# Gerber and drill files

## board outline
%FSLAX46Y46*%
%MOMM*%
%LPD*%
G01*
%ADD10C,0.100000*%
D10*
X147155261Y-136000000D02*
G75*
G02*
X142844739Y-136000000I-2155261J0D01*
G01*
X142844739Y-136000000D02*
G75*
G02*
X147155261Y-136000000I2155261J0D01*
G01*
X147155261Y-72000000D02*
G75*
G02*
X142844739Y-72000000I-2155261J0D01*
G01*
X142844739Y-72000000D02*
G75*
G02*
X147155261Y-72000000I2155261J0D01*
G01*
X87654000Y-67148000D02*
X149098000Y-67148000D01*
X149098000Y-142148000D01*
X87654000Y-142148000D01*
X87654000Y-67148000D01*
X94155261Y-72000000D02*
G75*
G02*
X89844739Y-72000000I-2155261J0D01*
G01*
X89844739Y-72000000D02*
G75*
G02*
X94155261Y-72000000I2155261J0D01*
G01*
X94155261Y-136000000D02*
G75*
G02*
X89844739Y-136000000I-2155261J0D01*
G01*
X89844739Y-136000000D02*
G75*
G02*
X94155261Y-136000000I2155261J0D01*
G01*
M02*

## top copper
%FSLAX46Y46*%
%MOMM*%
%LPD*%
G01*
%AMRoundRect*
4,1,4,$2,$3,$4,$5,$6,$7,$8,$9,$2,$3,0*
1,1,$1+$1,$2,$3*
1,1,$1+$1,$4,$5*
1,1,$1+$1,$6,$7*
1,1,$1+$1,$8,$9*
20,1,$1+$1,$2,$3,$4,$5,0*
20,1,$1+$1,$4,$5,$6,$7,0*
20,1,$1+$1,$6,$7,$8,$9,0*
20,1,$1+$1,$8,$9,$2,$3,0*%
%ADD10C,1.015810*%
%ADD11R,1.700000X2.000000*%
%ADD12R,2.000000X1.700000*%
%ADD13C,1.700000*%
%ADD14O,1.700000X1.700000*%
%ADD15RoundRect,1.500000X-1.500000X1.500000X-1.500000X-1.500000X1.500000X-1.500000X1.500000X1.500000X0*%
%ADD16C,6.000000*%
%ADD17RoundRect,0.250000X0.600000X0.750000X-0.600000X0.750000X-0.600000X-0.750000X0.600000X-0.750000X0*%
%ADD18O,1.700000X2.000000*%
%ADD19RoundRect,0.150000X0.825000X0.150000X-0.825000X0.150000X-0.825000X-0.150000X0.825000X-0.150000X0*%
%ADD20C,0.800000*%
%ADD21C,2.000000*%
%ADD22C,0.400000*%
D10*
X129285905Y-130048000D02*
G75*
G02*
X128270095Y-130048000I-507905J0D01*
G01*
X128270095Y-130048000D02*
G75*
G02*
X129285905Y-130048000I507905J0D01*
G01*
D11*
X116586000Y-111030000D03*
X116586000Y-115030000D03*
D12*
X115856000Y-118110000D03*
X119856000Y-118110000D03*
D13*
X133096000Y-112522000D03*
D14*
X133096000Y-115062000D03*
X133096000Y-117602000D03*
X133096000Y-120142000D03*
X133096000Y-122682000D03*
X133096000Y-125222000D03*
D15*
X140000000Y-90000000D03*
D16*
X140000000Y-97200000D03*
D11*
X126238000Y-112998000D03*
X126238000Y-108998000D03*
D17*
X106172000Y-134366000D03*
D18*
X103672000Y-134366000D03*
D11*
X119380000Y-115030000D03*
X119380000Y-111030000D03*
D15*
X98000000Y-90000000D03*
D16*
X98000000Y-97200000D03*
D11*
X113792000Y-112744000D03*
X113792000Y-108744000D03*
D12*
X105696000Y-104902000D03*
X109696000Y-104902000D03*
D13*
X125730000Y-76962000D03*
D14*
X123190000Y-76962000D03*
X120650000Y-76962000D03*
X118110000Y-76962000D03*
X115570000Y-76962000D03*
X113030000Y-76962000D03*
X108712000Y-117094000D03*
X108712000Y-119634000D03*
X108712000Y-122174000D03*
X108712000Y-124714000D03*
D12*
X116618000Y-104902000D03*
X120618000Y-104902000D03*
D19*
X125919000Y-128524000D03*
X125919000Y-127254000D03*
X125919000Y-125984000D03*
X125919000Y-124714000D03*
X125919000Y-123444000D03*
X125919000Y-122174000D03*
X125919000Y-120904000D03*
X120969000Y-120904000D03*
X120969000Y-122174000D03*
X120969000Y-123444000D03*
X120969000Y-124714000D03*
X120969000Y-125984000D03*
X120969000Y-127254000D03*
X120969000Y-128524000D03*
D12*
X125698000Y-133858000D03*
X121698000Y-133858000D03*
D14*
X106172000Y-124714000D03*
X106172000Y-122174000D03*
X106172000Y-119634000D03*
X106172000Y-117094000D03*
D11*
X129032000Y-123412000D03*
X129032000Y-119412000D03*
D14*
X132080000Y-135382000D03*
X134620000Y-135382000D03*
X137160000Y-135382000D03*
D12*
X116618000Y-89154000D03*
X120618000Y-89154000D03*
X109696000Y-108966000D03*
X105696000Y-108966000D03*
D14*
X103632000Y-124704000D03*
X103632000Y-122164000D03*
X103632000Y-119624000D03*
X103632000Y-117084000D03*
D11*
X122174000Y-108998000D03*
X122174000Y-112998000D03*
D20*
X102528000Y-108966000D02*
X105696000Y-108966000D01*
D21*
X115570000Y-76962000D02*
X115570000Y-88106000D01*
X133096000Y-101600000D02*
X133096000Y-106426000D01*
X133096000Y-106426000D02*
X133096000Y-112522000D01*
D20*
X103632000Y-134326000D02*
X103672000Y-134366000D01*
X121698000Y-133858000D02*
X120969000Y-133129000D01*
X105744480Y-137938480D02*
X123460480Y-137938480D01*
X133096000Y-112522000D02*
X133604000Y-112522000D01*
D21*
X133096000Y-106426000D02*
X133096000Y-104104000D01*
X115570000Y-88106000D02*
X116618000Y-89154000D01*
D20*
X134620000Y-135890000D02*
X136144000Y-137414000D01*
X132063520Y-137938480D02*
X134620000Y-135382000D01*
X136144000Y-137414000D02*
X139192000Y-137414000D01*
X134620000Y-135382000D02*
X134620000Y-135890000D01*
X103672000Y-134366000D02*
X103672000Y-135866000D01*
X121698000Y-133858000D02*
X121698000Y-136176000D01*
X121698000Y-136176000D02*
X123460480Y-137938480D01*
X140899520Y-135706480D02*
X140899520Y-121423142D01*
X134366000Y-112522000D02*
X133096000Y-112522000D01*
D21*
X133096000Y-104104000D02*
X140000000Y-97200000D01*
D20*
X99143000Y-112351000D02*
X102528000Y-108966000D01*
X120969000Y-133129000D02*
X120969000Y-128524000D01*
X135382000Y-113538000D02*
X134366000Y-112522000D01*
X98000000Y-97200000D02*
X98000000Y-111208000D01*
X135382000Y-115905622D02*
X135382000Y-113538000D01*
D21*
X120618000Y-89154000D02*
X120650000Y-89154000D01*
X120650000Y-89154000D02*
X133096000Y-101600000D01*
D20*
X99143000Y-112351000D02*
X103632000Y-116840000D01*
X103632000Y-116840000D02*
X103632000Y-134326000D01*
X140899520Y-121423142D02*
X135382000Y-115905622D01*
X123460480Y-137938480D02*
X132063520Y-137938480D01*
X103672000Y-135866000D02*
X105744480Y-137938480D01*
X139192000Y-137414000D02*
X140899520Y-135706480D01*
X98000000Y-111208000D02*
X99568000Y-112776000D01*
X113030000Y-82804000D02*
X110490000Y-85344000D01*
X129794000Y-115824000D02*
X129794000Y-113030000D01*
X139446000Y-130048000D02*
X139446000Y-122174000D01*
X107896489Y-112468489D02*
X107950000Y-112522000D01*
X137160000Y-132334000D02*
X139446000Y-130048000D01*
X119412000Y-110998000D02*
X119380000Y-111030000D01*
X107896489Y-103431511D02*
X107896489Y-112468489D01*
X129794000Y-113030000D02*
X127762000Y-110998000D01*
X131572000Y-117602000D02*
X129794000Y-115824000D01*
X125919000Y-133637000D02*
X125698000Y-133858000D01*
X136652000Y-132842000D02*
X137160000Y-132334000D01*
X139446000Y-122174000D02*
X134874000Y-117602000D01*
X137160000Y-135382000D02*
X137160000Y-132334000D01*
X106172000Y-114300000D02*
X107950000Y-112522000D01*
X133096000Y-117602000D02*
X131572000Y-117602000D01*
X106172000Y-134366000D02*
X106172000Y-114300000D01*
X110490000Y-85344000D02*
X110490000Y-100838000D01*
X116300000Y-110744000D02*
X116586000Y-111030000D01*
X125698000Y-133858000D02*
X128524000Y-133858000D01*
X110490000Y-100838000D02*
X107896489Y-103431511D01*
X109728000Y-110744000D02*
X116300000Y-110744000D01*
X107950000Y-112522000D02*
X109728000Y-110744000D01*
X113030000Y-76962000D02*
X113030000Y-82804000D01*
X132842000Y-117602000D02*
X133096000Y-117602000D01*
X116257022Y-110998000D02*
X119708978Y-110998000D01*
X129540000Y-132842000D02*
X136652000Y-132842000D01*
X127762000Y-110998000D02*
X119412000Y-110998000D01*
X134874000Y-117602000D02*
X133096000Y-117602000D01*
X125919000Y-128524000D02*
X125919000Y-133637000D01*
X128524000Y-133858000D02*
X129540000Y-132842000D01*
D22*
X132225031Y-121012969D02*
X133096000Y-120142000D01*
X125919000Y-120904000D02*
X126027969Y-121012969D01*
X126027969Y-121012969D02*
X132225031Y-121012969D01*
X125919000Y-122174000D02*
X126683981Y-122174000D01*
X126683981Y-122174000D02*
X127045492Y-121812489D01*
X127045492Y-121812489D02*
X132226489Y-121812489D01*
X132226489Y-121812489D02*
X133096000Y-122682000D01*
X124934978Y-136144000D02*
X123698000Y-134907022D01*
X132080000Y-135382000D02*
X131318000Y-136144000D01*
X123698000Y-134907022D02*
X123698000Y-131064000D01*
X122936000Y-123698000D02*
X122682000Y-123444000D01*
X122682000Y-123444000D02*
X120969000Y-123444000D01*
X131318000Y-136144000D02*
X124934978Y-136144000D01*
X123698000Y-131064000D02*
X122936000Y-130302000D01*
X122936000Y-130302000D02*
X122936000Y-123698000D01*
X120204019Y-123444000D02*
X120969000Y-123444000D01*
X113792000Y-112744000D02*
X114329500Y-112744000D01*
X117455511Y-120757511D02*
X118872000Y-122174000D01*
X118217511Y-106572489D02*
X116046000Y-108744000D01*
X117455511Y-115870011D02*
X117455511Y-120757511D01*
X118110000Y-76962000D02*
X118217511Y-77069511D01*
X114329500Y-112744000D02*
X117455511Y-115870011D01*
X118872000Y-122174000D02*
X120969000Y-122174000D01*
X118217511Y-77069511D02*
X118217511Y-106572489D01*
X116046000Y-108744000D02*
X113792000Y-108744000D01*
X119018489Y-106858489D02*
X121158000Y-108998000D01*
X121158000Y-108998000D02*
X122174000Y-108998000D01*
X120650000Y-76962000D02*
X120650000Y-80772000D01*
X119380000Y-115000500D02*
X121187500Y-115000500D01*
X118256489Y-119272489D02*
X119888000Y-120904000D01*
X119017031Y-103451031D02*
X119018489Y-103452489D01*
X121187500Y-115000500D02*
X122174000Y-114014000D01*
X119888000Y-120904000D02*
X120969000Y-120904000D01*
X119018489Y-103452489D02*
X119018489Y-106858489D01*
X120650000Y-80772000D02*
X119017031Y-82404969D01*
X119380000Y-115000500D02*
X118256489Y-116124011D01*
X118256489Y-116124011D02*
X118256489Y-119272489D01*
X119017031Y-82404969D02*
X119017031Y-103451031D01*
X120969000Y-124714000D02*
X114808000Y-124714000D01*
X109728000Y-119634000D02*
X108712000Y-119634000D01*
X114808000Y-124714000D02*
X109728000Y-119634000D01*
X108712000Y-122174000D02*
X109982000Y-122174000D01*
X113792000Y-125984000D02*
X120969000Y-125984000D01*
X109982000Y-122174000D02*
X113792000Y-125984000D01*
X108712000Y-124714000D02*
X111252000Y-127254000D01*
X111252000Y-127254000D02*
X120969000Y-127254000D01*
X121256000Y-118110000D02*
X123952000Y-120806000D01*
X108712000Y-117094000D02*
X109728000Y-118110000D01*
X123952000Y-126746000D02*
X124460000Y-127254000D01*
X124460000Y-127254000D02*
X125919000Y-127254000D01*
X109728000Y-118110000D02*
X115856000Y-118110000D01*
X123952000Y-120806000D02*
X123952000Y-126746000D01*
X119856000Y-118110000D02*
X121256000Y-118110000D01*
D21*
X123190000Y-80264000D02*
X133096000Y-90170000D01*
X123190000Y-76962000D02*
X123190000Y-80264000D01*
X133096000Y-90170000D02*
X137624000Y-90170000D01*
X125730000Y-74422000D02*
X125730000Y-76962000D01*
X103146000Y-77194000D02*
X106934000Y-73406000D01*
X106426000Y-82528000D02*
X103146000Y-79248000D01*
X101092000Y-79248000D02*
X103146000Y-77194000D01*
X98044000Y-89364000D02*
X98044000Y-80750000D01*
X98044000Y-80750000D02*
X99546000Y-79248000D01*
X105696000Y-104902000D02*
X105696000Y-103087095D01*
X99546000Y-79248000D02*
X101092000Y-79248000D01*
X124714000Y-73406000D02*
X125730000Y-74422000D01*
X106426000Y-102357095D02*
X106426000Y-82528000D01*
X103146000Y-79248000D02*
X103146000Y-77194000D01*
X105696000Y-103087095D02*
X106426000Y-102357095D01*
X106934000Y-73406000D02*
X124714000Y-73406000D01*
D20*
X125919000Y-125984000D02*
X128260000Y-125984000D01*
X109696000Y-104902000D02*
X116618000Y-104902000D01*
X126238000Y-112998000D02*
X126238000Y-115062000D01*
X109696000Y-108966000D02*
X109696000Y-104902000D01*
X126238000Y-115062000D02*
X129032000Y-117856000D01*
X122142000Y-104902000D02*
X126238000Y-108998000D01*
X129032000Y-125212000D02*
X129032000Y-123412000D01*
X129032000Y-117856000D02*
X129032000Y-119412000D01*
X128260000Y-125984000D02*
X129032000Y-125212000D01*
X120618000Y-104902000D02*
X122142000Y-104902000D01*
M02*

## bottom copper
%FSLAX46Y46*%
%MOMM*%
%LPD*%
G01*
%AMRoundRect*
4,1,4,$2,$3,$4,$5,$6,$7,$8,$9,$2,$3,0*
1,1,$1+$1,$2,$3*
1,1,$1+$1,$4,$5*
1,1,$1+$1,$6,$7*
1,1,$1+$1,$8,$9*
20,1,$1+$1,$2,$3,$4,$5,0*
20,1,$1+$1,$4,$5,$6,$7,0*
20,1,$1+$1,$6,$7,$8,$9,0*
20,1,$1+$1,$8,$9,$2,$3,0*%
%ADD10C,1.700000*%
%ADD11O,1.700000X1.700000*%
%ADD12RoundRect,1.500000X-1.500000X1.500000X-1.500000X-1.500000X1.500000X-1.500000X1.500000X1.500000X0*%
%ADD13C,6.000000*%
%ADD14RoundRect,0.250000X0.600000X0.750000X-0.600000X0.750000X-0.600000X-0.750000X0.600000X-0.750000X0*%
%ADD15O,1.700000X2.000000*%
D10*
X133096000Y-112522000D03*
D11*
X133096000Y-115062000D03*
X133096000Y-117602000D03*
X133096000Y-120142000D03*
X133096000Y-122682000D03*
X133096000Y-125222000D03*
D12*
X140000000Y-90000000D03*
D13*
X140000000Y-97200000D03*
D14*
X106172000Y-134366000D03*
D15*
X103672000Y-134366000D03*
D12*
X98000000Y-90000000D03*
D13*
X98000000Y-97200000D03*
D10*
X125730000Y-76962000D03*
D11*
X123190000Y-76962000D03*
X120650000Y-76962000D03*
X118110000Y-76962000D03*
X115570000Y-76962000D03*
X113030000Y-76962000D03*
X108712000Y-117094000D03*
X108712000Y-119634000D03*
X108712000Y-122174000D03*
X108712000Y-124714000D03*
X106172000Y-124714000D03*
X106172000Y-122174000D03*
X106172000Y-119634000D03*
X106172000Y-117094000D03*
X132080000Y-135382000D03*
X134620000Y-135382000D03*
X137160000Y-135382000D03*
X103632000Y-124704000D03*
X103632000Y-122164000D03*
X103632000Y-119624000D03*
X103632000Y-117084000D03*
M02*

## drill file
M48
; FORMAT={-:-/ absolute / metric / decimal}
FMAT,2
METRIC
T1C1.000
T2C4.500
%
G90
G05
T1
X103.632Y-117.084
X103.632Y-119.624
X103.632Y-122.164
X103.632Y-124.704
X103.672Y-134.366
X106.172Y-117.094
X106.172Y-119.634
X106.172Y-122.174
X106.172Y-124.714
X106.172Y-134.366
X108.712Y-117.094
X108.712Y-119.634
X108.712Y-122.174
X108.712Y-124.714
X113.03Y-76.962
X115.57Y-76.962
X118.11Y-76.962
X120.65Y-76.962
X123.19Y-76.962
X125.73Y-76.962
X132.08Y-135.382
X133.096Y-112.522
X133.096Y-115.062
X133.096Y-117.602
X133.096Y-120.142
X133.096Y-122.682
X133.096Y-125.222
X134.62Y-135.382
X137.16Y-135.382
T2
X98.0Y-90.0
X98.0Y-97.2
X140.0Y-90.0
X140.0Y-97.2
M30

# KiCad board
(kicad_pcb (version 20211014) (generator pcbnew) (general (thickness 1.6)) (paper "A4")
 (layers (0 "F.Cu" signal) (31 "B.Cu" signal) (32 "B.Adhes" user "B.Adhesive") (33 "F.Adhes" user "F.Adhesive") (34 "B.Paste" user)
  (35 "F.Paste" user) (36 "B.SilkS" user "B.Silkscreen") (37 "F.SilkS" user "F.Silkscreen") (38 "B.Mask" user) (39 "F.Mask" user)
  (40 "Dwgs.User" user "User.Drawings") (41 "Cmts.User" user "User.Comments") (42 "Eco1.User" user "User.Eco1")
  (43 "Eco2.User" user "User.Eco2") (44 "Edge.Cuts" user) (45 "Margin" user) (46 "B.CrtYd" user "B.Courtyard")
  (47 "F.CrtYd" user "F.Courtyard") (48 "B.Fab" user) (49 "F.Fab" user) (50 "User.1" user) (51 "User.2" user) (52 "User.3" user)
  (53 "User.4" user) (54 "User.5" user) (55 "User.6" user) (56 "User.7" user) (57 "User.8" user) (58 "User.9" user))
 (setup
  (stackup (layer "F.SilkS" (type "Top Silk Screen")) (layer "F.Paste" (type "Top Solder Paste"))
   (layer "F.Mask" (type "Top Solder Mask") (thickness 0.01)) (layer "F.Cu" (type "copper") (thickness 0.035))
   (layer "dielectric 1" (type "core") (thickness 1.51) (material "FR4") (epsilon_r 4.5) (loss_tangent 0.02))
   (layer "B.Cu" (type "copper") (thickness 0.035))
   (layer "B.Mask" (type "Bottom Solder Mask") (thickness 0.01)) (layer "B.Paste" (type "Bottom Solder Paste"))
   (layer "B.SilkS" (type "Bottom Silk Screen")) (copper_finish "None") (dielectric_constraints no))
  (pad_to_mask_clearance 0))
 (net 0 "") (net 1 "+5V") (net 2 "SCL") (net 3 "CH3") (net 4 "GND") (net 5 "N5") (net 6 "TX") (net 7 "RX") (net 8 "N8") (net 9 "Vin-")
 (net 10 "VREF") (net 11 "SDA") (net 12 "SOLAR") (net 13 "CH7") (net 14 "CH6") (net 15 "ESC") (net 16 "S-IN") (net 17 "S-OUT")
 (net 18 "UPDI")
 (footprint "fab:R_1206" (layer "F.Cu") (at 116.586 113.03 -90)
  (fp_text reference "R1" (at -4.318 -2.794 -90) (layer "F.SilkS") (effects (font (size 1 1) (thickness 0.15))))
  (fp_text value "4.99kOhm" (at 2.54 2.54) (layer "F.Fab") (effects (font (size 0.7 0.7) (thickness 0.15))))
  (pad "1" smd rect locked (at -2 0 270) (size 2 1.7) (layers "F.Cu" "F.Paste" "F.Mask") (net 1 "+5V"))
  (pad "2" smd rect locked (at 2 0 270) (size 2 1.7) (layers "F.Cu" "F.Paste" "F.Mask") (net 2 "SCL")))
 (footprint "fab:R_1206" (layer "F.Cu") (at 117.856 118.11)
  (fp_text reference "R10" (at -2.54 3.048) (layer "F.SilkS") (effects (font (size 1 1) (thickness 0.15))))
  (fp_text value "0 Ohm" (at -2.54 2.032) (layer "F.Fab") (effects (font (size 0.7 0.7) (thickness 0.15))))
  (pad "1" smd rect locked (at -2 0) (size 2 1.7) (layers "F.Cu" "F.Paste" "F.Mask") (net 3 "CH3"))
  (pad "2" smd rect locked (at 2 0) (size 2 1.7) (layers "F.Cu" "F.Paste" "F.Mask") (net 3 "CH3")))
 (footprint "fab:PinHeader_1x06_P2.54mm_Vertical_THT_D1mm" (layer "F.Cu") (at 133.096 112.522)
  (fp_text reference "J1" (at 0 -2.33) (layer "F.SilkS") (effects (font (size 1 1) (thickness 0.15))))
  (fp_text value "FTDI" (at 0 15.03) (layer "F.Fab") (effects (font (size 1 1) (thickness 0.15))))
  (pad "1" thru_hole circle locked (at 0 0) (size 1.7 1.7) (drill 1) (layers *.Cu *.Mask) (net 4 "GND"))
  (pad "2" thru_hole oval locked (at 0 2.54) (size 1.7 1.7) (drill 1) (layers *.Cu *.Mask) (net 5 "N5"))
  (pad "3" thru_hole oval locked (at 0 5.08) (size 1.7 1.7) (drill 1) (layers *.Cu *.Mask) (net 1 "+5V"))
  (pad "4" thru_hole oval locked (at 0 7.62) (size 1.7 1.7) (drill 1) (layers *.Cu *.Mask) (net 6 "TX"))
  (pad "5" thru_hole oval locked (at 0 10.16) (size 1.7 1.7) (drill 1) (layers *.Cu *.Mask) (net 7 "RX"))
  (pad "6" thru_hole oval locked (at 0 12.7) (size 1.7 1.7) (drill 1) (layers *.Cu *.Mask) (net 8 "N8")))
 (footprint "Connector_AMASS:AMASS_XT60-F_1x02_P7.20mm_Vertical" (layer "F.Cu") (at 140 90 -90)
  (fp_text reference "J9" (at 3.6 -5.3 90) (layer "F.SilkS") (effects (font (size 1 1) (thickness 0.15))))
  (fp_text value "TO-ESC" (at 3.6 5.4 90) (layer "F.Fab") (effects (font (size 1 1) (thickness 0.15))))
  (pad "1" thru_hole roundrect (at 0 0 270) (size 6 6) (drill 4.5) (layers *.Cu *.Mask) (roundrect_rratio 0.25) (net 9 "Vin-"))
  (pad "2" thru_hole circle (at 7.2 0 270) (size 6 6) (drill 4.5) (layers *.Cu *.Mask) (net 4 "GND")))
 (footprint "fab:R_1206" (layer "F.Cu") (at 126.238 110.998 90)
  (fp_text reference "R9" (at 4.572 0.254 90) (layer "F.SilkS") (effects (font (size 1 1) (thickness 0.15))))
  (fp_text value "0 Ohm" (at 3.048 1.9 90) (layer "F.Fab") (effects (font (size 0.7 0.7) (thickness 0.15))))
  (pad "1" smd rect locked (at -2 0 90) (size 2 1.7) (layers "F.Cu" "F.Paste" "F.Mask") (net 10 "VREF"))
  (pad "2" smd rect locked (at 2 0 90) (size 2 1.7) (layers "F.Cu" "F.Paste" "F.Mask") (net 10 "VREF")))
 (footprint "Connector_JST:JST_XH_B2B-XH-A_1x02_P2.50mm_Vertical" (layer "F.Cu") (at 106.172 134.366 180)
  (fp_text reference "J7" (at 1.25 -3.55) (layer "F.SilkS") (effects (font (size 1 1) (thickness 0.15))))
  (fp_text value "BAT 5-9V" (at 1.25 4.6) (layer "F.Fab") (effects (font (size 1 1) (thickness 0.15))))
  (pad "1" thru_hole roundrect (at 0 0 180) (size 1.7 2) (drill 1) (layers *.Cu *.Mask) (roundrect_rratio 0.1470588235) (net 1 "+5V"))
  (pad "2" thru_hole oval (at 2.5 0 180) (size 1.7 2) (drill 1) (layers *.Cu *.Mask) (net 4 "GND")))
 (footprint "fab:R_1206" (layer "F.Cu") (at 119.38 113.03 90)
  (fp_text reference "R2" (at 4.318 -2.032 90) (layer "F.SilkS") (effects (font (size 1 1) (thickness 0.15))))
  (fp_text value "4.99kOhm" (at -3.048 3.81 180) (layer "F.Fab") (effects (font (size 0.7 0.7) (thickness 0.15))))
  (pad "1" smd rect locked (at -2 0 90) (size 2 1.7) (layers "F.Cu" "F.Paste" "F.Mask") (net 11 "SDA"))
  (pad "2" smd rect locked (at 2 0 90) (size 2 1.7) (layers "F.Cu" "F.Paste" "F.Mask") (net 1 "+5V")))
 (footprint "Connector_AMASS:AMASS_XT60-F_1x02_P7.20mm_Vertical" (layer "F.Cu") (at 98 90 -90)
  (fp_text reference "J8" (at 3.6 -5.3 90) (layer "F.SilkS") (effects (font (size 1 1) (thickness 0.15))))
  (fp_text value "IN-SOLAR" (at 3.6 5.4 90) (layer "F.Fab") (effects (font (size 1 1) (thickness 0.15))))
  (pad "1" thru_hole roundrect (at 0 0 270) (size 6 6) (drill 4.5) (layers *.Cu *.Mask) (roundrect_rratio 0.25) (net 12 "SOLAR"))
  (pad "2" thru_hole circle (at 7.2 0 270) (size 6 6) (drill 4.5) (layers *.Cu *.Mask) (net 4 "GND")))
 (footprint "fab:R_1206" (layer "F.Cu") (at 113.792 110.744 90)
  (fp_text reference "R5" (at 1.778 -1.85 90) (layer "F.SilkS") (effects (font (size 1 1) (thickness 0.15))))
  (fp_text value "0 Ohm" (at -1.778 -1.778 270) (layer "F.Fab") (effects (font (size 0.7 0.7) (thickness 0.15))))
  (pad "1" smd rect locked (at -2 0 90) (size 2 1.7) (layers "F.Cu" "F.Paste" "F.Mask") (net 2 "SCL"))
  (pad "2" smd rect locked (at 2 0 90) (size 2 1.7) (layers "F.Cu" "F.Paste" "F.Mask") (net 2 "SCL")))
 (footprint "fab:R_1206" (layer "F.Cu") (at 107.696 104.902)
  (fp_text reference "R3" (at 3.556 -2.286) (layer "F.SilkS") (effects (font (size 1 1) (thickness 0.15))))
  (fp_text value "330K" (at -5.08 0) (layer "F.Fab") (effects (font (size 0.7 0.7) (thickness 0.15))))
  (pad "1" smd rect locked (at -2 0) (size 2 1.7) (layers "F.Cu" "F.Paste" "F.Mask") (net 12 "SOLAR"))
  (pad "2" smd rect locked (at 2 0) (size 2 1.7) (layers "F.Cu" "F.Paste" "F.Mask") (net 10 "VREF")))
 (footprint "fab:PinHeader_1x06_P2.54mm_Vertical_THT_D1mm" (layer "F.Cu") (at 125.73 76.962 -90)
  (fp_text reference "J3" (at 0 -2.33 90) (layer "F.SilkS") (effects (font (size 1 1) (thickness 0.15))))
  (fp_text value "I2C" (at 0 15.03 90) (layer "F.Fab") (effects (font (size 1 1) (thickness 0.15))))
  (pad "1" thru_hole circle locked (at 0 0 270) (size 1.7 1.7) (drill 1) (layers *.Cu *.Mask) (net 12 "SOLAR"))
  (pad "2" thru_hole oval locked (at 0 2.54 270) (size 1.7 1.7) (drill 1) (layers *.Cu *.Mask) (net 9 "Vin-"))
  (pad "3" thru_hole oval locked (at 0 5.08 270) (size 1.7 1.7) (drill 1) (layers *.Cu *.Mask) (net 11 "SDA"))
  (pad "4" thru_hole oval locked (at 0 7.62 270) (size 1.7 1.7) (drill 1) (layers *.Cu *.Mask) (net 2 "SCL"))
  (pad "5" thru_hole oval locked (at 0 10.16 270) (size 1.7 1.7) (drill 1) (layers *.Cu *.Mask) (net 4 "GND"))
  (pad "6" thru_hole oval locked (at 0 12.7 270) (size 1.7 1.7) (drill 1) (layers *.Cu *.Mask) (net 1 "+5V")))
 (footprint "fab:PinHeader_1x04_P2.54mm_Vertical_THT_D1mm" (layer "F.Cu") (at 108.712 117.094)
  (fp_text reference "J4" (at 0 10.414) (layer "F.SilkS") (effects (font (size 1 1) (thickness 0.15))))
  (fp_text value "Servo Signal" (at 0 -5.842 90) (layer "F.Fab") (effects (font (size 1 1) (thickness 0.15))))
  (pad "1" thru_hole oval locked (at 0 0) (size 1.7 1.7) (drill 1) (layers *.Cu *.Mask) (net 3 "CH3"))
  (pad "2" thru_hole oval locked (at 0 2.54) (size 1.7 1.7) (drill 1) (layers *.Cu *.Mask) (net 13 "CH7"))
  (pad "3" thru_hole oval locked (at 0 5.08) (size 1.7 1.7) (drill 1) (layers *.Cu *.Mask) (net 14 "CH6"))
  (pad "4" thru_hole oval locked (at 0 7.62) (size 1.7 1.7) (drill 1) (layers *.Cu *.Mask) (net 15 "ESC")))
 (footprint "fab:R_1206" (layer "F.Cu") (at 118.618 104.902)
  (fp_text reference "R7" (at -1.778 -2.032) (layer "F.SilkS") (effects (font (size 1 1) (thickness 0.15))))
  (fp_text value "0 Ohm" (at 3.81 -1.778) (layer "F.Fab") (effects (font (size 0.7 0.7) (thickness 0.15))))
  (pad "1" smd rect locked (at -2 0) (size 2 1.7) (layers "F.Cu" "F.Paste" "F.Mask") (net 10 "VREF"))
  (pad "2" smd rect locked (at 2 0) (size 2 1.7) (layers "F.Cu" "F.Paste" "F.Mask") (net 10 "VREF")))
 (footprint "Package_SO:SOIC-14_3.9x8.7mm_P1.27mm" (layer "F.Cu") (at 123.444 124.714 180)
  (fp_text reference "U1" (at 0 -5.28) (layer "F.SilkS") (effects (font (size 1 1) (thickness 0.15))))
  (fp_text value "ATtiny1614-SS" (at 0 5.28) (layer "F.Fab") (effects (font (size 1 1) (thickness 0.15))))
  (pad "1" smd roundrect (at -2.475 -3.81 180) (size 1.95 0.6) (layers "F.Cu" "F.Paste" "F.Mask") (roundrect_rratio 0.25) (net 1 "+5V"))
  (pad "2" smd roundrect (at -2.475 -2.54 180) (size 1.95 0.6) (layers "F.Cu" "F.Paste" "F.Mask") (roundrect_rratio 0.25) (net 3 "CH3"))
  (pad "3" smd roundrect (at -2.475 -1.27 180) (size 1.95 0.6) (layers "F.Cu" "F.Paste" "F.Mask") (roundrect_rratio 0.25) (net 10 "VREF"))
  (pad "4" smd roundrect (at -2.475 0 180) (size 1.95 0.6) (layers "F.Cu" "F.Paste" "F.Mask") (roundrect_rratio 0.25) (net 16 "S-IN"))
  (pad "5" smd roundrect (at -2.475 1.27 180) (size 1.95 0.6) (layers "F.Cu" "F.Paste" "F.Mask") (roundrect_rratio 0.25) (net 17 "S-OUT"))
  (pad "6" smd roundrect (at -2.475 2.54 180) (size 1.95 0.6) (layers "F.Cu" "F.Paste" "F.Mask") (roundrect_rratio 0.25) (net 7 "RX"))
  (pad "7" smd roundrect (at -2.475 3.81 180) (size 1.95 0.6) (layers "F.Cu" "F.Paste" "F.Mask") (roundrect_rratio 0.25) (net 6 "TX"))
  (pad "8" smd roundrect (at 2.475 3.81 180) (size 1.95 0.6) (layers "F.Cu" "F.Paste" "F.Mask") (roundrect_rratio 0.25) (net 11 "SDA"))
  (pad "9" smd roundrect (at 2.475 2.54 180) (size 1.95 0.6) (layers "F.Cu" "F.Paste" "F.Mask") (roundrect_rratio 0.25) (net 2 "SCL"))
  (pad "10" smd roundrect (at 2.475 1.27 180) (size 1.95 0.6) (layers "F.Cu" "F.Paste" "F.Mask") (roundrect_rratio 0.25) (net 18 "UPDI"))
  (pad "11" smd roundrect (at 2.475 0 180) (size 1.95 0.6) (layers "F.Cu" "F.Paste" "F.Mask") (roundrect_rratio 0.25) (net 13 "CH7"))
  (pad "12" smd roundrect (at 2.475 -1.27 180) (size 1.95 0.6) (layers "F.Cu" "F.Paste" "F.Mask") (roundrect_rratio 0.25) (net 14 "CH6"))
  (pad "13" smd roundrect (at 2.475 -2.54 180) (size 1.95 0.6) (layers "F.Cu" "F.Paste" "F.Mask") (roundrect_rratio 0.25) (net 15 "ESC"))
  (pad "14" smd roundrect (at 2.475 -3.81 180) (size 1.95 0.6) (layers "F.Cu" "F.Paste" "F.Mask") (roundrect_rratio 0.25) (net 4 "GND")))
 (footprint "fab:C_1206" (layer "F.Cu") (at 123.698 133.858 180)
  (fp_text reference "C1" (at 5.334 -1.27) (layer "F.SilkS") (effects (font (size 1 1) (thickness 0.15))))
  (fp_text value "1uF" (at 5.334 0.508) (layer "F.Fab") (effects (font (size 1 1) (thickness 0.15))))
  (pad "1" smd rect locked (at -2 0 180) (size 2 1.7) (layers "F.Cu" "F.Paste" "F.Mask") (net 1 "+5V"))
  (pad "2" smd rect locked (at 2 0 180) (size 2 1.7) (layers "F.Cu" "F.Paste" "F.Mask") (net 4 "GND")))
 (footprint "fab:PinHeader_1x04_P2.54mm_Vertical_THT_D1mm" (layer "F.Cu") (at 106.172 124.714 180)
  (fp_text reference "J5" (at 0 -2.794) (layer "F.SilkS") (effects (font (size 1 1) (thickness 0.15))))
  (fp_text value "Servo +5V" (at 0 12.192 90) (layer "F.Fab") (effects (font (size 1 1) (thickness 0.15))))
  (pad "1" thru_hole oval locked (at 0 0 180) (size 1.7 1.7) (drill 1) (layers *.Cu *.Mask) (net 1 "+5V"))
  (pad "2" thru_hole oval locked (at 0 2.54 180) (size 1.7 1.7) (drill 1) (layers *.Cu *.Mask) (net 1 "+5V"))
  (pad "3" thru_hole oval locked (at 0 5.08 180) (size 1.7 1.7) (drill 1) (layers *.Cu *.Mask) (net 1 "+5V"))
  (pad "4" thru_hole oval locked (at 0 7.62 180) (size 1.7 1.7) (drill 1) (layers *.Cu *.Mask) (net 1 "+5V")))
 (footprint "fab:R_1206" (layer "F.Cu") (at 129.032 121.412 90)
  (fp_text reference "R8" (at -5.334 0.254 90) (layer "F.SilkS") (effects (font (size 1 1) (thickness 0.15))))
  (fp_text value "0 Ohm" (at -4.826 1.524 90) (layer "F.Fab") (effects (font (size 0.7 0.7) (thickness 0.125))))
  (pad "1" smd rect locked (at -2 0 90) (size 2 1.7) (layers "F.Cu" "F.Paste" "F.Mask") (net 10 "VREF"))
  (pad "2" smd rect locked (at 2 0 90) (size 2 1.7) (layers "F.Cu" "F.Paste" "F.Mask") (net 10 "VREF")))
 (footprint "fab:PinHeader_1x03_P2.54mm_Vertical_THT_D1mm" (layer "F.Cu") (at 132.08 135.382 90)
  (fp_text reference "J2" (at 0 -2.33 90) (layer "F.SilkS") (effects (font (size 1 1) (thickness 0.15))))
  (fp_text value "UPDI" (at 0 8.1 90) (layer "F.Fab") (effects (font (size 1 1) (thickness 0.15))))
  (pad "1" thru_hole oval locked (at 0 0 90) (size 1.7 1.7) (drill 1) (layers *.Cu *.Mask) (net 18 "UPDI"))
  (pad "2" thru_hole oval locked (at 0 2.54 90) (size 1.7 1.7) (drill 1) (layers *.Cu *.Mask) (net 4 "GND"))
  (pad "3" thru_hole oval locked (at 0 5.08 90) (size 1.7 1.7) (drill 1) (layers *.Cu *.Mask) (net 1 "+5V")))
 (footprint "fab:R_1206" (layer "F.Cu") (at 118.618 89.154)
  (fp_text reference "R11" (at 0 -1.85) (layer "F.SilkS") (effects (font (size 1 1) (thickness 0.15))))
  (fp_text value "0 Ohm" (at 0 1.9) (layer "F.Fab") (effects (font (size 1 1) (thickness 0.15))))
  (pad "1" smd rect locked (at -2 0) (size 2 1.7) (layers "F.Cu" "F.Paste" "F.Mask") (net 4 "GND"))
  (pad "2" smd rect locked (at 2 0) (size 2 1.7) (layers "F.Cu" "F.Paste" "F.Mask") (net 4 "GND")))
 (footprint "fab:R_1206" (layer "F.Cu") (at 107.696 108.966 180)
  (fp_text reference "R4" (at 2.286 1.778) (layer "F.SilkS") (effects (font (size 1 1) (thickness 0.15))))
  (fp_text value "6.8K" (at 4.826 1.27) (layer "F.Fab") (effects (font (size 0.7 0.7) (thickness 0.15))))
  (pad "1" smd rect locked (at -2 0 180) (size 2 1.7) (layers "F.Cu" "F.Paste" "F.Mask") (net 10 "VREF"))
  (pad "2" smd rect locked (at 2 0 180) (size 2 1.7) (layers "F.Cu" "F.Paste" "F.Mask") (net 4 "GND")))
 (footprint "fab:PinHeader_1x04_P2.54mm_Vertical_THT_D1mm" (layer "F.Cu") (at 103.632 124.704 180)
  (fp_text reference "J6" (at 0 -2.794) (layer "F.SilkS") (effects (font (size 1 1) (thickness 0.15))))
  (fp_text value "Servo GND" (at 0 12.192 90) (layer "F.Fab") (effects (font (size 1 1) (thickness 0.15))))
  (pad "1" thru_hole oval locked (at 0 0 180) (size 1.7 1.7) (drill 1) (layers *.Cu *.Mask) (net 4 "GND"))
  (pad "2" thru_hole oval locked (at 0 2.54 180) (size 1.7 1.7) (drill 1) (layers *.Cu *.Mask) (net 4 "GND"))
  (pad "3" thru_hole oval locked (at 0 5.08 180) (size 1.7 1.7) (drill 1) (layers *.Cu *.Mask) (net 4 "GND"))
  (pad "4" thru_hole oval locked (at 0 7.62 180) (size 1.7 1.7) (drill 1) (layers *.Cu *.Mask) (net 4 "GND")))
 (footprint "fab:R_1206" (layer "F.Cu") (at 122.174 110.998 -90)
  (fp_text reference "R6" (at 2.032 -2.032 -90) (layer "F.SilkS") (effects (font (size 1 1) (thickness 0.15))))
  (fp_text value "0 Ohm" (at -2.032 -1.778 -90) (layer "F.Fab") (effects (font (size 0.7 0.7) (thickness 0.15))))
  (pad "1" smd rect locked (at -2 0 270) (size 2 1.7) (layers "F.Cu" "F.Paste" "F.Mask") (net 11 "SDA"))
  (pad "2" smd rect locked (at 2 0 270) (size 2 1.7) (layers "F.Cu" "F.Paste" "F.Mask") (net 11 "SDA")))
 (gr_circle (center 128.778 130.048) (end 129.69381 130.048) (layer "F.Cu") (width 0.2) (fill solid))
 (gr_circle (center 145 136) (end 147.155261 136) (layer "Edge.Cuts") (width 0.1) (fill none))
 (gr_circle (center 145 72) (end 147.155261 72) (layer "Edge.Cuts") (width 0.1) (fill none))
 (gr_rect (start 87.654 67.148) (end 149.098 142.148) (layer "Edge.Cuts") (width 0.1) (fill none))
 (gr_circle (center 92 72) (end 94.155261 72) (layer "Edge.Cuts") (width 0.1) (fill none))
 (gr_circle (center 92 136) (end 94.155261 136) (layer "Edge.Cuts") (width 0.1) (fill none))
 (segment (start 102.528 108.966) (end 105.696 108.966) (width 0.8) (layer "F.Cu") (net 4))
 (segment (start 115.57 76.962) (end 115.57 88.106) (width 2) (layer "F.Cu") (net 4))
 (segment (start 133.096 101.6) (end 133.096 106.426) (width 2) (layer "F.Cu") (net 4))
 (segment (start 133.096 106.426) (end 133.096 112.522) (width 2) (layer "F.Cu") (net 4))
 (segment (start 103.632 134.326) (end 103.672 134.366) (width 0.8) (layer "F.Cu") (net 4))
 (segment (start 121.698 133.858) (end 120.969 133.129) (width 0.8) (layer "F.Cu") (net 4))
 (segment (start 105.74448 137.93848) (end 123.46048 137.93848) (width 0.8) (layer "F.Cu") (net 4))
 (segment (start 133.096 112.522) (end 133.604 112.522) (width 0.8) (layer "F.Cu") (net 4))
 (segment (start 133.096 106.426) (end 133.096 104.104) (width 2) (layer "F.Cu") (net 4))
 (segment (start 115.57 88.106) (end 116.618 89.154) (width 2) (layer "F.Cu") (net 4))
 (segment (start 134.62 135.89) (end 136.144 137.414) (width 0.8) (layer "F.Cu") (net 4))
 (segment (start 132.06352 137.93848) (end 134.62 135.382) (width 0.8) (layer "F.Cu") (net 4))
 (segment (start 136.144 137.414) (end 139.192 137.414) (width 0.8) (layer "F.Cu") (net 4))
 (segment (start 134.62 135.382) (end 134.62 135.89) (width 0.8) (layer "F.Cu") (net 4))
 (segment (start 103.672 134.366) (end 103.672 135.866) (width 0.8) (layer "F.Cu") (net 4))
 (segment (start 121.698 133.858) (end 121.698 136.176) (width 0.8) (layer "F.Cu") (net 4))
 (segment (start 121.698 136.176) (end 123.46048 137.93848) (width 0.8) (layer "F.Cu") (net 4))
 (segment (start 140.89952 135.70648) (end 140.89952 121.423142) (width 0.8) (layer "F.Cu") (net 4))
 (segment (start 134.366 112.522) (end 133.096 112.522) (width 0.8) (layer "F.Cu") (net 4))
 (segment (start 133.096 104.104) (end 140 97.2) (width 2) (layer "F.Cu") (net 4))
 (segment (start 99.143 112.351) (end 102.528 108.966) (width 0.8) (layer "F.Cu") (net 4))
 (segment (start 120.969 133.129) (end 120.969 128.524) (width 0.8) (layer "F.Cu") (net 4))
 (segment (start 135.382 113.538) (end 134.366 112.522) (width 0.8) (layer "F.Cu") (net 4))
 (segment (start 98 97.2) (end 98 111.208) (width 0.8) (layer "F.Cu") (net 4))
 (segment (start 135.382 115.905622) (end 135.382 113.538) (width 0.8) (layer "F.Cu") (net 4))
 (segment (start 120.618 89.154) (end 120.65 89.154) (width 2) (layer "F.Cu") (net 4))
 (segment (start 120.65 89.154) (end 133.096 101.6) (width 2) (layer "F.Cu") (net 4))
 (segment (start 99.143 112.351) (end 103.632 116.84) (width 0.8) (layer "F.Cu") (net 4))
 (segment (start 103.632 116.84) (end 103.632 134.326) (width 0.8) (layer "F.Cu") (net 4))
 (segment (start 140.89952 121.423142) (end 135.382 115.905622) (width 0.8) (layer "F.Cu") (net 4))
 (segment (start 123.46048 137.93848) (end 132.06352 137.93848) (width 0.8) (layer "F.Cu") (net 4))
 (segment (start 103.672 135.866) (end 105.74448 137.93848) (width 0.8) (layer "F.Cu") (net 4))
 (segment (start 139.192 137.414) (end 140.89952 135.70648) (width 0.8) (layer "F.Cu") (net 4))
 (segment (start 98 111.208) (end 99.568 112.776) (width 0.8) (layer "F.Cu") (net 4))
 (segment (start 113.03 82.804) (end 110.49 85.344) (width 0.8) (layer "F.Cu") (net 1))
 (segment (start 129.794 115.824) (end 129.794 113.03) (width 0.8) (layer "F.Cu") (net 1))
 (segment (start 139.446 130.048) (end 139.446 122.174) (width 0.8) (layer "F.Cu") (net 1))
 (segment (start 107.896489 112.468489) (end 107.95 112.522) (width 0.8) (layer "F.Cu") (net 1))
 (segment (start 137.16 132.334) (end 139.446 130.048) (width 0.8) (layer "F.Cu") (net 1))
 (segment (start 119.412 110.998) (end 119.38 111.03) (width 0.8) (layer "F.Cu") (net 1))
 (segment (start 107.896489 103.431511) (end 107.896489 112.468489) (width 0.8) (layer "F.Cu") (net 1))
 (segment (start 129.794 113.03) (end 127.762 110.998) (width 0.8) (layer "F.Cu") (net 1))
 (segment (start 131.572 117.602) (end 129.794 115.824) (width 0.8) (layer "F.Cu") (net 1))
 (segment (start 125.919 133.637) (end 125.698 133.858) (width 0.8) (layer "F.Cu") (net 1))
 (segment (start 136.652 132.842) (end 137.16 132.334) (width 0.8) (layer "F.Cu") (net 1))
 (segment (start 139.446 122.174) (end 134.874 117.602) (width 0.8) (layer "F.Cu") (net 1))
 (segment (start 137.16 135.382) (end 137.16 132.334) (width 0.8) (layer "F.Cu") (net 1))
 (segment (start 106.172 114.3) (end 107.95 112.522) (width 0.8) (layer "F.Cu") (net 1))
 (segment (start 133.096 117.602) (end 131.572 117.602) (width 0.8) (layer "F.Cu") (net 1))
 (segment (start 106.172 134.366) (end 106.172 114.3) (width 0.8) (layer "F.Cu") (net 1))
 (segment (start 110.49 85.344) (end 110.49 100.838) (width 0.8) (layer "F.Cu") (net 1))
 (segment (start 116.3 110.744) (end 116.586 111.03) (width 0.8) (layer "F.Cu") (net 1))
 (segment (start 125.698 133.858) (end 128.524 133.858) (width 0.8) (layer "F.Cu") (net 1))
 (segment (start 110.49 100.838) (end 107.896489 103.431511) (width 0.8) (layer "F.Cu") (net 1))
 (segment (start 109.728 110.744) (end 116.3 110.744) (width 0.8) (layer "F.Cu") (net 1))
 (segment (start 107.95 112.522) (end 109.728 110.744) (width 0.8) (layer "F.Cu") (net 1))
 (segment (start 113.03 76.962) (end 113.03 82.804) (width 0.8) (layer "F.Cu") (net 1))
 (segment (start 132.842 117.602) (end 133.096 117.602) (width 0.8) (layer "F.Cu") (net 1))
 (segment (start 116.257022 110.998) (end 119.708978 110.998) (width 0.8) (layer "F.Cu") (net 1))
 (segment (start 129.54 132.842) (end 136.652 132.842) (width 0.8) (layer "F.Cu") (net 1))
 (segment (start 127.762 110.998) (end 119.412 110.998) (width 0.8) (layer "F.Cu") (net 1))
 (segment (start 134.874 117.602) (end 133.096 117.602) (width 0.8) (layer "F.Cu") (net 1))
 (segment (start 125.919 128.524) (end 125.919 133.637) (width 0.8) (layer "F.Cu") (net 1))
 (segment (start 128.524 133.858) (end 129.54 132.842) (width 0.8) (layer "F.Cu") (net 1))
 (segment (start 132.225031 121.012969) (end 133.096 120.142) (width 0.4) (layer "F.Cu") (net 6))
 (segment (start 125.919 120.904) (end 126.027969 121.012969) (width 0.4) (layer "F.Cu") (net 6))
 (segment (start 126.027969 121.012969) (end 132.225031 121.012969) (width 0.4) (layer "F.Cu") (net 6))
 (segment (start 125.919 122.174) (end 126.683981 122.174) (width 0.4) (layer "F.Cu") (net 7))
 (segment (start 126.683981 122.174) (end 127.045492 121.812489) (width 0.4) (layer "F.Cu") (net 7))
 (segment (start 127.045492 121.812489) (end 132.226489 121.812489) (width 0.4) (layer "F.Cu") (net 7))
 (segment (start 132.226489 121.812489) (end 133.096 122.682) (width 0.4) (layer "F.Cu") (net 7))
 (segment (start 124.934978 136.144) (end 123.698 134.907022) (width 0.4) (layer "F.Cu") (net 18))
 (segment (start 132.08 135.382) (end 131.318 136.144) (width 0.4) (layer "F.Cu") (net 18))
 (segment (start 123.698 134.907022) (end 123.698 131.064) (width 0.4) (layer "F.Cu") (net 18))
 (segment (start 122.936 123.698) (end 122.682 123.444) (width 0.4) (layer "F.Cu") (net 18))
 (segment (start 122.682 123.444) (end 120.969 123.444) (width 0.4) (layer "F.Cu") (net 18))
 (segment (start 131.318 136.144) (end 124.934978 136.144) (width 0.4) (layer "F.Cu") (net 18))
 (segment (start 123.698 131.064) (end 122.936 130.302) (width 0.4) (layer "F.Cu") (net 18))
 (segment (start 122.936 130.302) (end 122.936 123.698) (width 0.4) (layer "F.Cu") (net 18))
 (segment (start 120.204019 123.444) (end 120.969 123.444) (width 0.4) (layer "F.Cu") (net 18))
 (segment (start 113.792 112.744) (end 114.3295 112.744) (width 0.4) (layer "F.Cu") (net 2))
 (segment (start 117.455511 120.757511) (end 118.872 122.174) (width 0.4) (layer "F.Cu") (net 2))
 (segment (start 118.217511 106.572489) (end 116.046 108.744) (width 0.4) (layer "F.Cu") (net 2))
 (segment (start 117.455511 115.870011) (end 117.455511 120.757511) (width 0.4) (layer "F.Cu") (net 2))
 (segment (start 118.11 76.962) (end 118.217511 77.069511) (width 0.4) (layer "F.Cu") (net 2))
 (segment (start 114.3295 112.744) (end 117.455511 115.870011) (width 0.4) (layer "F.Cu") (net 2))
 (segment (start 118.872 122.174) (end 120.969 122.174) (width 0.4) (layer "F.Cu") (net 2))
 (segment (start 118.217511 77.069511) (end 118.217511 106.572489) (width 0.4) (layer "F.Cu") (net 2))
 (segment (start 116.046 108.744) (end 113.792 108.744) (width 0.4) (layer "F.Cu") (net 2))
 (segment (start 119.018489 106.858489) (end 121.158 108.998) (width 0.4) (layer "F.Cu") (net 11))
 (segment (start 121.158 108.998) (end 122.174 108.998) (width 0.4) (layer "F.Cu") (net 11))
 (segment (start 120.65 76.962) (end 120.65 80.772) (width 0.4) (layer "F.Cu") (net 11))
 (segment (start 119.38 115.0005) (end 121.1875 115.0005) (width 0.4) (layer "F.Cu") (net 11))
 (segment (start 118.256489 119.272489) (end 119.888 120.904) (width 0.4) (layer "F.Cu") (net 11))
 (segment (start 119.017031 103.451031) (end 119.018489 103.452489) (width 0.4) (layer "F.Cu") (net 11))
 (segment (start 121.1875 115.0005) (end 122.174 114.014) (width 0.4) (layer "F.Cu") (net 11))
 (segment (start 119.888 120.904) (end 120.969 120.904) (width 0.4) (layer "F.Cu") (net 11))
 (segment (start 119.018489 103.452489) (end 119.018489 106.858489) (width 0.4) (layer "F.Cu") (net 11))
 (segment (start 120.65 80.772) (end 119.017031 82.404969) (width 0.4) (layer "F.Cu") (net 11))
 (segment (start 119.38 115.0005) (end 118.256489 116.124011) (width 0.4) (layer "F.Cu") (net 11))
 (segment (start 118.256489 116.124011) (end 118.256489 119.272489) (width 0.4) (layer "F.Cu") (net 11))
 (segment (start 119.017031 82.404969) (end 119.017031 103.451031) (width 0.4) (layer "F.Cu") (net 11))
 (segment (start 120.969 124.714) (end 114.808 124.714) (width 0.4) (layer "F.Cu") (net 13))
 (segment (start 109.728 119.634) (end 108.712 119.634) (width 0.4) (layer "F.Cu") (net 13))
 (segment (start 114.808 124.714) (end 109.728 119.634) (width 0.4) (layer "F.Cu") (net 13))
 (segment (start 108.712 122.174) (end 109.982 122.174) (width 0.4) (layer "F.Cu") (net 14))
 (segment (start 113.792 125.984) (end 120.969 125.984) (width 0.4) (layer "F.Cu") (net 14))
 (segment (start 109.982 122.174) (end 113.792 125.984) (width 0.4) (layer "F.Cu") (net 14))
 (segment (start 108.712 124.714) (end 111.252 127.254) (width 0.4) (layer "F.Cu") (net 15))
 (segment (start 111.252 127.254) (end 120.969 127.254) (width 0.4) (layer "F.Cu") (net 15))
 (segment (start 121.256 118.11) (end 123.952 120.806) (width 0.4) (layer "F.Cu") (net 3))
 (segment (start 108.712 117.094) (end 109.728 118.11) (width 0.4) (layer "F.Cu") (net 3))
 (segment (start 123.952 126.746) (end 124.46 127.254) (width 0.4) (layer "F.Cu") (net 3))
 (segment (start 124.46 127.254) (end 125.919 127.254) (width 0.4) (layer "F.Cu") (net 3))
 (segment (start 109.728 118.11) (end 115.856 118.11) (width 0.4) (layer "F.Cu") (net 3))
 (segment (start 123.952 120.806) (end 123.952 126.746) (width 0.4) (layer "F.Cu") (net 3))
 (segment (start 119.856 118.11) (end 121.256 118.11) (width 0.4) (layer "F.Cu") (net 3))
 (segment (start 123.19 80.264) (end 133.096 90.17) (width 2) (layer "F.Cu") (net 9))
 (segment (start 123.19 76.962) (end 123.19 80.264) (width 2) (layer "F.Cu") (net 9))
 (segment (start 133.096 90.17) (end 137.624 90.17) (width 2) (layer "F.Cu") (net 9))
 (segment (start 125.73 74.422) (end 125.73 76.962) (width 2) (layer "F.Cu") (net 12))
 (segment (start 103.146 77.194) (end 106.934 73.406) (width 2) (layer "F.Cu") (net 12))
 (segment (start 106.426 82.528) (end 103.146 79.248) (width 2) (layer "F.Cu") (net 12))
 (segment (start 101.092 79.248) (end 103.146 77.194) (width 2) (layer "F.Cu") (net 12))
 (segment (start 98.044 89.364) (end 98.044 80.75) (width 2) (layer "F.Cu") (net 12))
 (segment (start 98.044 80.75) (end 99.546 79.248) (width 2) (layer "F.Cu") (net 12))
 (segment (start 105.696 104.902) (end 105.696 103.087095) (width 2) (layer "F.Cu") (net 12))
 (segment (start 99.546 79.248) (end 101.092 79.248) (width 2) (layer "F.Cu") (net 12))
 (segment (start 124.714 73.406) (end 125.73 74.422) (width 2) (layer "F.Cu") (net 12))
 (segment (start 106.426 102.357095) (end 106.426 82.528) (width 2) (layer "F.Cu") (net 12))
 (segment (start 103.146 79.248) (end 103.146 77.194) (width 2) (layer "F.Cu") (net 12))
 (segment (start 105.696 103.087095) (end 106.426 102.357095) (width 2) (layer "F.Cu") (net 12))
 (segment (start 106.934 73.406) (end 124.714 73.406) (width 2) (layer "F.Cu") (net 12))
 (segment (start 125.919 125.984) (end 128.26 125.984) (width 0.8) (layer "F.Cu") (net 10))
 (segment (start 109.696 104.902) (end 116.618 104.902) (width 0.8) (layer "F.Cu") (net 10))
 (segment (start 126.238 112.998) (end 126.238 115.062) (width 0.8) (layer "F.Cu") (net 10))
 (segment (start 109.696 108.966) (end 109.696 104.902) (width 0.8) (layer "F.Cu") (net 10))
 (segment (start 126.238 115.062) (end 129.032 117.856) (width 0.8) (layer "F.Cu") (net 10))
 (segment (start 122.142 104.902) (end 126.238 108.998) (width 0.8) (layer "F.Cu") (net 10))
 (segment (start 129.032 125.212) (end 129.032 123.412) (width 0.8) (layer "F.Cu") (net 10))
 (segment (start 129.032 117.856) (end 129.032 119.412) (width 0.8) (layer "F.Cu") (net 10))
 (segment (start 128.26 125.984) (end 129.032 125.212) (width 0.8) (layer "F.Cu") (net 10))
 (segment (start 120.618 104.902) (end 122.142 104.902) (width 0.8) (layer "F.Cu") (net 10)))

